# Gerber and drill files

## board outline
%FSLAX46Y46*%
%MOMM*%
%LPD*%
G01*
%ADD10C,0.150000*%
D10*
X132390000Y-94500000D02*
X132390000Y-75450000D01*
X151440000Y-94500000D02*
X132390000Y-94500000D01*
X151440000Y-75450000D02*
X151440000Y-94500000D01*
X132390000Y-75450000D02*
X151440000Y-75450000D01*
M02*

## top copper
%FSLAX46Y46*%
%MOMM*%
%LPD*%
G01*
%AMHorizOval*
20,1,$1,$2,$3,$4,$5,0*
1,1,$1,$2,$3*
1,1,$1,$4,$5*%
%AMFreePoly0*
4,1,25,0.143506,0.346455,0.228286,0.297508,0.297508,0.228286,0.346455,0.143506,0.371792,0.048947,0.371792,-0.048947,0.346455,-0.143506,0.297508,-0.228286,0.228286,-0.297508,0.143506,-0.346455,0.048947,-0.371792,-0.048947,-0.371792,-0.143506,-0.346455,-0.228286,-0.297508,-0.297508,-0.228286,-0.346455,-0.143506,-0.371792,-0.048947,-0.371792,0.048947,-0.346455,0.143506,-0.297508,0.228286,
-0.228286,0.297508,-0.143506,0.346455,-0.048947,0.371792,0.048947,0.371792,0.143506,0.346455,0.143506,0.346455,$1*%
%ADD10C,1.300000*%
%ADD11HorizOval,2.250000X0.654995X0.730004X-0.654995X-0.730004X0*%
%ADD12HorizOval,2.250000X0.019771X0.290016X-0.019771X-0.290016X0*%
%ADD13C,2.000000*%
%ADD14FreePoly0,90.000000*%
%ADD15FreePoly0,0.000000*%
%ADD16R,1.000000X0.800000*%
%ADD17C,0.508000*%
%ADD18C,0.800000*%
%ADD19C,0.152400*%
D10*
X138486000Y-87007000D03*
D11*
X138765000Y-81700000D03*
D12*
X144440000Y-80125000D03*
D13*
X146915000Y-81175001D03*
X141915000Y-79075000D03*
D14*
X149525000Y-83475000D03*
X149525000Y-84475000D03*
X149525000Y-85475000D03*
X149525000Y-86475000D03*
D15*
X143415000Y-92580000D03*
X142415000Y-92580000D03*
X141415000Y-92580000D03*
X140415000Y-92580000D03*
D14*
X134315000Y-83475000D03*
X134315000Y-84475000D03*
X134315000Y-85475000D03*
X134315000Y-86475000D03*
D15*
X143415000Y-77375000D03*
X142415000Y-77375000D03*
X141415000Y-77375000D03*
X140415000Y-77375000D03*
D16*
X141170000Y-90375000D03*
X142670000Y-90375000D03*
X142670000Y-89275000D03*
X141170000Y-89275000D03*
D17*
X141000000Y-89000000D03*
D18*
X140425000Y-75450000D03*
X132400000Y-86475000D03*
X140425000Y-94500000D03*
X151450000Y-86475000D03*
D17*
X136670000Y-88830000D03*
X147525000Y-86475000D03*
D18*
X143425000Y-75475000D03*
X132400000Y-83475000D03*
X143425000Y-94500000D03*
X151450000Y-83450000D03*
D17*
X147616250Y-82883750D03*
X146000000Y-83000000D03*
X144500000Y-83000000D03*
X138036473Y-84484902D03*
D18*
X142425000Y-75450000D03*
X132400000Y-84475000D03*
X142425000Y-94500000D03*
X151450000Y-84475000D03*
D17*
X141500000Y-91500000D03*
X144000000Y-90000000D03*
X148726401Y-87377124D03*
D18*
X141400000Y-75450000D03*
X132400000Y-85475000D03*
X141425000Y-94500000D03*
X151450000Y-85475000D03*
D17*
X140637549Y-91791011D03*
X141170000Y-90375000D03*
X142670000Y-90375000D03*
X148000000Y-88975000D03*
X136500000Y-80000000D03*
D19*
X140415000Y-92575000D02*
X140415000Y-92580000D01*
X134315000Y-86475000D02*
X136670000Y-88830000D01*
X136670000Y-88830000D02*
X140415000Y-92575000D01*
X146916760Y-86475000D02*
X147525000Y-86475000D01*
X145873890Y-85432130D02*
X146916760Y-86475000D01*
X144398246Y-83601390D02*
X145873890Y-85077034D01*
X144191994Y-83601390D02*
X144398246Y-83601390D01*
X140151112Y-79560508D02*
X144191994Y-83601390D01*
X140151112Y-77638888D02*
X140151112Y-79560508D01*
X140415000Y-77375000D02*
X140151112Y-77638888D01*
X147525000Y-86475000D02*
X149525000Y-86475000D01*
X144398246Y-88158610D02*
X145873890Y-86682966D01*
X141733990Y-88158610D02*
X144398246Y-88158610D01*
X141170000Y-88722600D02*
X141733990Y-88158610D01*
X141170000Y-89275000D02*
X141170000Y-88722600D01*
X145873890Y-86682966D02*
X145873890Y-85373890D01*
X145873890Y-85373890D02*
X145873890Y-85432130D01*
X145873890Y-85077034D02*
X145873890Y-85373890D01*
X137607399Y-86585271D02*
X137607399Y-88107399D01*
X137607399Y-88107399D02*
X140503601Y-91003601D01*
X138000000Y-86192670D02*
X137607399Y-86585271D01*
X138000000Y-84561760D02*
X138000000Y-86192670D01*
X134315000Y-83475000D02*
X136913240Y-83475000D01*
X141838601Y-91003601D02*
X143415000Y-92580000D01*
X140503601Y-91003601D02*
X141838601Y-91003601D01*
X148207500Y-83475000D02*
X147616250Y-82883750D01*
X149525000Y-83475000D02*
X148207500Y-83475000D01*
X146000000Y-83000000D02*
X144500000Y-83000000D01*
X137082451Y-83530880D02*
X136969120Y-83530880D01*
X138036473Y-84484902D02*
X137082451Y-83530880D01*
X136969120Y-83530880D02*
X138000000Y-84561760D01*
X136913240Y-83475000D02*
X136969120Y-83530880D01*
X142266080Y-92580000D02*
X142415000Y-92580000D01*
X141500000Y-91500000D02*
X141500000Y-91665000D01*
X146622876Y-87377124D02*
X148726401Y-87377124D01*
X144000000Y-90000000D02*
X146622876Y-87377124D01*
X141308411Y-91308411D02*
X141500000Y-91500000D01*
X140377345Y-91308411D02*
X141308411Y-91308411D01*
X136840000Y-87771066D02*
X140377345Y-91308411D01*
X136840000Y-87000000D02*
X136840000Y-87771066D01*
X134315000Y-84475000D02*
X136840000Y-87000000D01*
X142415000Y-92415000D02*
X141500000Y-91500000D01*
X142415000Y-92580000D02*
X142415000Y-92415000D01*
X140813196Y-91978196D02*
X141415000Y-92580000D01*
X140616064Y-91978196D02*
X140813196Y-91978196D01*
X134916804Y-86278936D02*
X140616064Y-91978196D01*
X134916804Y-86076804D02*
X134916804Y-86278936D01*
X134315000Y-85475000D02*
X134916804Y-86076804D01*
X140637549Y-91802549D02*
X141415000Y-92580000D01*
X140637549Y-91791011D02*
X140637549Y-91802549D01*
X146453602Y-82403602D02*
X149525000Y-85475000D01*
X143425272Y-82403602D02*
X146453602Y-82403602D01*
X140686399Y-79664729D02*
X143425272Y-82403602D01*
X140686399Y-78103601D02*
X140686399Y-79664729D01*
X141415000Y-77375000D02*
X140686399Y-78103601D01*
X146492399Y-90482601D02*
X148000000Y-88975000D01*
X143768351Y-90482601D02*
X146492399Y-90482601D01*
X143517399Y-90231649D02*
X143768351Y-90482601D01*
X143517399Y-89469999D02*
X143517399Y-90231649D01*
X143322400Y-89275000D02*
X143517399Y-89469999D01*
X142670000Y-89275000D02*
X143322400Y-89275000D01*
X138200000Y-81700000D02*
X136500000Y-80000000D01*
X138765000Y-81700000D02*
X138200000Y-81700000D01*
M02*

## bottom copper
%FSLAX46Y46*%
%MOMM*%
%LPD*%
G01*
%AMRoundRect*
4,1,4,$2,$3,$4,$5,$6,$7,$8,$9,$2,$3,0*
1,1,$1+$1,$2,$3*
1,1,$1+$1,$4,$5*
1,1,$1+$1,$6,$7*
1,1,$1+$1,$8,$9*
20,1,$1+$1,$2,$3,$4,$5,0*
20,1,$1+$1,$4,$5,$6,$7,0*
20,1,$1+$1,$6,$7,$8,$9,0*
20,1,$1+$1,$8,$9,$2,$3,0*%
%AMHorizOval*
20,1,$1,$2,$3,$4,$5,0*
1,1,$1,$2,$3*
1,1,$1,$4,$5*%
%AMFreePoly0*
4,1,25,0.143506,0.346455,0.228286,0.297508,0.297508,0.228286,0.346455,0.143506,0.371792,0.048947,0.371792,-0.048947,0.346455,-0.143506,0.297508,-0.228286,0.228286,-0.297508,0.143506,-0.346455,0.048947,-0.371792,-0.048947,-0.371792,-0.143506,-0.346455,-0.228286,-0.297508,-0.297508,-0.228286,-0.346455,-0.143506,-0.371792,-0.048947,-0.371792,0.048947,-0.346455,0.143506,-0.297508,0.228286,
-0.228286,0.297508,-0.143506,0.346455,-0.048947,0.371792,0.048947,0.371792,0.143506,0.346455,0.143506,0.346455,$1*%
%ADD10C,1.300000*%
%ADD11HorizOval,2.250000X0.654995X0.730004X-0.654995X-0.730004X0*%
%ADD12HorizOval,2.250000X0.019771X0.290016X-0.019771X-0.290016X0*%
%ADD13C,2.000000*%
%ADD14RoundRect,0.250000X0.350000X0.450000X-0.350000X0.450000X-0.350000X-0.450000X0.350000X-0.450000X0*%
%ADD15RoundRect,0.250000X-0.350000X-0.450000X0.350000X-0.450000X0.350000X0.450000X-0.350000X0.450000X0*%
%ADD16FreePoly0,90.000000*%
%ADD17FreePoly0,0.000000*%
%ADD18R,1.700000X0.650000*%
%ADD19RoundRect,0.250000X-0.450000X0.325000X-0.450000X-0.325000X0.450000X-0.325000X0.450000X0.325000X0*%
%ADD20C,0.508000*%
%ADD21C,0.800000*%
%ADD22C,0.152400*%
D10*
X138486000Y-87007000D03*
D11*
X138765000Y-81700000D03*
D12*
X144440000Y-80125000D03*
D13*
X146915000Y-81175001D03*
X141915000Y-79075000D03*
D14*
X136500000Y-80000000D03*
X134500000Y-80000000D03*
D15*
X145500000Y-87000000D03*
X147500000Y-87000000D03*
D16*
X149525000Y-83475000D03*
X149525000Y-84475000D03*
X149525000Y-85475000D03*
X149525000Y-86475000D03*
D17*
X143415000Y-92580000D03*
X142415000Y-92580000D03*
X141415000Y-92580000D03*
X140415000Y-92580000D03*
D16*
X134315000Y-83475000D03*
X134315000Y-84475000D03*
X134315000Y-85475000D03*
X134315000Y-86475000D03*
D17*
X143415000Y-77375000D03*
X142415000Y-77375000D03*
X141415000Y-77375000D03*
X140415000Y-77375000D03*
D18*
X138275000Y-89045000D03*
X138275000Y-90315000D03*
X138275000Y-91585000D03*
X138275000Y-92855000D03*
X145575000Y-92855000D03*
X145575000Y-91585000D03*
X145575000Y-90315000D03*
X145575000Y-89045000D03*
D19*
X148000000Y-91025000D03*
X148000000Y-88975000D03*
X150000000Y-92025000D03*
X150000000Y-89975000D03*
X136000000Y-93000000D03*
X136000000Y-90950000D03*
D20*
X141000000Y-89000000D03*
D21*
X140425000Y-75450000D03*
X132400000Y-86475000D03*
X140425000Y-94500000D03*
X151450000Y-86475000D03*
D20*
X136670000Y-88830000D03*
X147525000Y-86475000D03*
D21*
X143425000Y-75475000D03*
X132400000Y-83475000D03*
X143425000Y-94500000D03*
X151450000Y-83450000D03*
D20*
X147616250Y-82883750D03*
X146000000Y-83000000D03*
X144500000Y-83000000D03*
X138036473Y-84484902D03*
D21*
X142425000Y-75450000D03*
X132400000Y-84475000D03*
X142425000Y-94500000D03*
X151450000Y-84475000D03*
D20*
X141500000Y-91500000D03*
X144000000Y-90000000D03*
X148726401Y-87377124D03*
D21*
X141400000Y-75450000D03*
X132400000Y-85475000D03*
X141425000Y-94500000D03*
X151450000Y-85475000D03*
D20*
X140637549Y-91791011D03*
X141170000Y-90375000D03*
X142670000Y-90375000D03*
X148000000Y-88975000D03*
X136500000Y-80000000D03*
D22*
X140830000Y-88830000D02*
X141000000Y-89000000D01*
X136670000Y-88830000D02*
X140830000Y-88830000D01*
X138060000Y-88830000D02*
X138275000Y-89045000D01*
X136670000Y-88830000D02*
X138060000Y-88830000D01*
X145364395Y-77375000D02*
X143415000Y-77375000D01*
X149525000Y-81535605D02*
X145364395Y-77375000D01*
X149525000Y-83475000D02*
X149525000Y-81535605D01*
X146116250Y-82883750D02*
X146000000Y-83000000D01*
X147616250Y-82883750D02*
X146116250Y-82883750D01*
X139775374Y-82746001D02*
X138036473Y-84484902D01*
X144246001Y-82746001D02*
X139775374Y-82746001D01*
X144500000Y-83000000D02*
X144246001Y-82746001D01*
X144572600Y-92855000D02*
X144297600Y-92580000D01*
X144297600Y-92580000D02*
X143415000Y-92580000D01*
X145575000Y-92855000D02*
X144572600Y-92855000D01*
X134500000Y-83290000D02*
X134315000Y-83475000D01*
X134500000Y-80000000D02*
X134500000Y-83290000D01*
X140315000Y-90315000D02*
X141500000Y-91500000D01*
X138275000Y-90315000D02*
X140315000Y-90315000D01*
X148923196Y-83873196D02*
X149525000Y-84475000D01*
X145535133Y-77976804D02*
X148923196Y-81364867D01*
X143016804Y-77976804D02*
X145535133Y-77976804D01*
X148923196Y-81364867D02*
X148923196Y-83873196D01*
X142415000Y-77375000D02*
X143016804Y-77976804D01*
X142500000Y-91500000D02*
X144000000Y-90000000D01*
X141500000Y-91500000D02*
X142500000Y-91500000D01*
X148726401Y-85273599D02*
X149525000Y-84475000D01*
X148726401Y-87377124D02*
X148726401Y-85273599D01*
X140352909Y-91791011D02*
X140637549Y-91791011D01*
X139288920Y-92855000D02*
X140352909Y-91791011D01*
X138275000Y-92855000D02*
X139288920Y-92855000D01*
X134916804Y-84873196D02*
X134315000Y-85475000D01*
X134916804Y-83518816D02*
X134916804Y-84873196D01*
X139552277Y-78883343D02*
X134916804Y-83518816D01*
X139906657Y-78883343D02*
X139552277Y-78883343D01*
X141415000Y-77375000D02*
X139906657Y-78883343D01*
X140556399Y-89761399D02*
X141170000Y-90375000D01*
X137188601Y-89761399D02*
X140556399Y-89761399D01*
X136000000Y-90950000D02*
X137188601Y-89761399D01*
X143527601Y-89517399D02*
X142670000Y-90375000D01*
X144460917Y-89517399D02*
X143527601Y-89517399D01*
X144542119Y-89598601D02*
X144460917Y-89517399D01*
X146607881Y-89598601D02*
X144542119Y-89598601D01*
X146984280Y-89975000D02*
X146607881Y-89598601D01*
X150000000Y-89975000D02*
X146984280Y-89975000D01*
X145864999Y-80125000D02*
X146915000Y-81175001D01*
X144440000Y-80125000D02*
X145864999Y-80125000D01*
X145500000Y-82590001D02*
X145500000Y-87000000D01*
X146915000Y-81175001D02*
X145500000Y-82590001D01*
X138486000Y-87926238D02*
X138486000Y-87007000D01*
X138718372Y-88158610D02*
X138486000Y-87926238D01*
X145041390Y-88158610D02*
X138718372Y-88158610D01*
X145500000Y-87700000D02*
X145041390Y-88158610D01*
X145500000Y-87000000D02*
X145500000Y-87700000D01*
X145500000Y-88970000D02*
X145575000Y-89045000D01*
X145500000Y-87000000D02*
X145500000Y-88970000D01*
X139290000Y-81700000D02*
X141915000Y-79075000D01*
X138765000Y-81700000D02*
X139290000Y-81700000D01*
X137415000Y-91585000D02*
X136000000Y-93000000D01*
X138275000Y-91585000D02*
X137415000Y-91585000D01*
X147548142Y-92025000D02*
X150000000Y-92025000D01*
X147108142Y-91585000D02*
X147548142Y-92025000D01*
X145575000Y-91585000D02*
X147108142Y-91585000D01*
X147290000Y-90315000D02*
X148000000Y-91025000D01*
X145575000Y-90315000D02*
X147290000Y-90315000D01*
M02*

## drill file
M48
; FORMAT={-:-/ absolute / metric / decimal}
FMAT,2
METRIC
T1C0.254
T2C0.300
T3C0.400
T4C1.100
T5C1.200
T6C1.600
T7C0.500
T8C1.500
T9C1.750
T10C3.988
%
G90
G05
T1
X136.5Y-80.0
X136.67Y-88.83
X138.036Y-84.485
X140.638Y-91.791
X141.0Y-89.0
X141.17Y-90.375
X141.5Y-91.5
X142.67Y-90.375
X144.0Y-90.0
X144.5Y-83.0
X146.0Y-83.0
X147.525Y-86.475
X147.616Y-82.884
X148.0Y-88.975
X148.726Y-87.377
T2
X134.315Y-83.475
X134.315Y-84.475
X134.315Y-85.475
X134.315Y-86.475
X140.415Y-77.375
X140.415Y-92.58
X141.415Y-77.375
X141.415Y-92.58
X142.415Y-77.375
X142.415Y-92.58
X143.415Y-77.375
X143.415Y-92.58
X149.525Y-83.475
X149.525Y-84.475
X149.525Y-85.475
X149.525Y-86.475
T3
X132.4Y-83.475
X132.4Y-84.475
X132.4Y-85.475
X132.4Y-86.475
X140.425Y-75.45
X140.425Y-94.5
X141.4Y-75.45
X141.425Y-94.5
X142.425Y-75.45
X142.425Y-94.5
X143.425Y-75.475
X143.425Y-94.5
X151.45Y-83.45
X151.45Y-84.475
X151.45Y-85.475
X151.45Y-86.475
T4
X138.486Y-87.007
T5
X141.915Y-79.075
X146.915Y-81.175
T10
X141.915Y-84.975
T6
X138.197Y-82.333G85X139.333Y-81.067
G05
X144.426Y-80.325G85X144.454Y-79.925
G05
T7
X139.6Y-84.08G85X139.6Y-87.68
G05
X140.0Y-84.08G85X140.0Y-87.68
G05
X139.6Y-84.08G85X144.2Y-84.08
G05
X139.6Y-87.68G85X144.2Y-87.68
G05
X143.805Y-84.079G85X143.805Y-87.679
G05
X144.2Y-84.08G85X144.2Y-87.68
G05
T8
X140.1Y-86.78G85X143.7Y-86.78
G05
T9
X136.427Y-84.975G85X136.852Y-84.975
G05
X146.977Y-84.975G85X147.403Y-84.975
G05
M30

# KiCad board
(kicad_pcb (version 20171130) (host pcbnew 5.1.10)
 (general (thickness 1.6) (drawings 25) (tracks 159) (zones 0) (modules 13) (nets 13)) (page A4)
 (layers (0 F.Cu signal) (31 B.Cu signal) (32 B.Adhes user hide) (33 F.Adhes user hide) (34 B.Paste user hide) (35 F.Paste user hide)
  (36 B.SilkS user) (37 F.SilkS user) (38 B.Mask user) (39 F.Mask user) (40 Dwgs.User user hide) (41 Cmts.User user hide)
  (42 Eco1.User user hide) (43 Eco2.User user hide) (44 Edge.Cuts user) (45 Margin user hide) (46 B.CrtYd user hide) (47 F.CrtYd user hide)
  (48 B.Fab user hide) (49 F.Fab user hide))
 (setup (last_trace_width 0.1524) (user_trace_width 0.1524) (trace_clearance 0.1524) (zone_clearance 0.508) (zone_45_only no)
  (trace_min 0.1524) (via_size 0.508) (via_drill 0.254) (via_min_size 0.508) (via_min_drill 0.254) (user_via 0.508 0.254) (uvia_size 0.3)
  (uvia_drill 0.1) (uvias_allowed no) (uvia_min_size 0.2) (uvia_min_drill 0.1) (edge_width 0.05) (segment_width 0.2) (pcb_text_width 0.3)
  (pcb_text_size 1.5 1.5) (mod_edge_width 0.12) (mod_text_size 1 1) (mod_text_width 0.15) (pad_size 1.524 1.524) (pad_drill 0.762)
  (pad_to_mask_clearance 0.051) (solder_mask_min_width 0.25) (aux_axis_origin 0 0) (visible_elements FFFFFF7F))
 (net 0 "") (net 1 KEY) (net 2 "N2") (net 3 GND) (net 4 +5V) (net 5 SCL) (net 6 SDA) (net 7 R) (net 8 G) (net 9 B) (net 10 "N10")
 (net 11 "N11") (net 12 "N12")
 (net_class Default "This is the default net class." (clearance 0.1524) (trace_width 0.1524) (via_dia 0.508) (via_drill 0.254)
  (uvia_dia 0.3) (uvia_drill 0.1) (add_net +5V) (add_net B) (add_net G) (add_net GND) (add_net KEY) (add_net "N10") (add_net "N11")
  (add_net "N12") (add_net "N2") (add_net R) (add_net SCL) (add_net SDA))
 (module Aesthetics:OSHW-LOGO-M (layer F.Cu) (at 147.5 91)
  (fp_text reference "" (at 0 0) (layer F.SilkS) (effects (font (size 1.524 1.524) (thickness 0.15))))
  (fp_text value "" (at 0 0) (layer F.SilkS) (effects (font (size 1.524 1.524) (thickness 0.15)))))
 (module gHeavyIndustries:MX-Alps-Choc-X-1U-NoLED (layer F.Cu) (at 141.915 84.975)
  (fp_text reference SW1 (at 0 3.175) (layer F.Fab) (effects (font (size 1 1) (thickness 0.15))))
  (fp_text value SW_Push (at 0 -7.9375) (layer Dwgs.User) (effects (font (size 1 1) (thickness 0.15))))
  (pad 1 thru_hole circle (at -3.429 2.032) (size 1.3 1.3) (drill 1.1) (layers *.Cu *.Mask) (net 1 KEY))
  (pad "" np_thru_hole oval (at -2.315 0.905) (size 0.5 4.1) (drill oval 0.5 4.1) (layers *.Cu *.Mask))
  (pad "" np_thru_hole oval (at 1.89 0.90416) (size 0.5 4.1) (drill oval 0.5 4.1) (layers *.Cu *.Mask))
  (pad "" np_thru_hole oval (at 2.285 0.905) (size 0.5 4.1) (drill oval 0.5 4.1) (layers *.Cu *.Mask))
  (pad "" np_thru_hole oval (at -0.015 2.705) (size 5.1 0.5) (drill oval 5.1 0.5) (layers *.Cu *.Mask))
  (pad "" np_thru_hole oval (at -0.015 -0.895) (size 5.1 0.5) (drill oval 5.1 0.5) (layers *.Cu *.Mask))
  (pad "" np_thru_hole oval (at -1.915 0.905) (size 0.5 4.1) (drill oval 0.5 4.1) (layers *.Cu *.Mask))
  (pad "" np_thru_hole oval (at -0.015 1.805) (size 5.1 1.5) (drill oval 5.1 1.5) (layers *.Cu *.Mask))
  (pad 2 thru_hole oval (at -3.15 -3.275 48.1) (size 4.211556 2.25) (drill oval 3.3 1.6) (layers *.Cu *.Mask) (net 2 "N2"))
  (pad 1 thru_hole oval (at 2.525 -4.85 86.1) (size 2.831378 2.25) (drill oval 2 1.6) (layers *.Cu *.Mask) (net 1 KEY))
  (pad "" np_thru_hole oval (at 5.275 0 90) (size 1.75 2.175) (drill oval 1.75 2.175) (layers *.Cu *.Mask))
  (pad "" np_thru_hole oval (at -5.275 0 90) (size 1.75 2.175) (drill oval 1.75 2.175) (layers *.Cu *.Mask))
  (pad "" np_thru_hole circle (at 0 0) (size 3.9878 3.9878) (drill 3.9878) (layers *.Cu *.Mask))
  (pad 1 thru_hole circle (at 5 -3.799999) (size 2 2) (drill 1.2) (layers *.Cu *.Mask) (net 1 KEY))
  (pad 2 thru_hole circle (at 0 -5.9) (size 2 2) (drill 1.2) (layers *.Cu *.Mask) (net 2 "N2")))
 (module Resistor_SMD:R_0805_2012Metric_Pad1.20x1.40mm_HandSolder (layer B.Cu) (at 135.5 80 180)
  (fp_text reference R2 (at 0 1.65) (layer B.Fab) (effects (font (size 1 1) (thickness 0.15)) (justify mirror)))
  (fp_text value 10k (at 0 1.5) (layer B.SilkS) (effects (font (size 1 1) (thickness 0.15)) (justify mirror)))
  (pad 1 smd roundrect (at -1 0 180) (size 1.2 1.4) (layers B.Cu B.Paste B.Mask) (roundrect_rratio 0.208333) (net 2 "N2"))
  (pad 2 smd roundrect (at 1 0 180) (size 1.2 1.4) (layers B.Cu B.Paste B.Mask) (roundrect_rratio 0.208333) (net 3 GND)))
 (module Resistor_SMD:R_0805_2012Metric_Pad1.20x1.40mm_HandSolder (layer B.Cu) (at 146.5 87)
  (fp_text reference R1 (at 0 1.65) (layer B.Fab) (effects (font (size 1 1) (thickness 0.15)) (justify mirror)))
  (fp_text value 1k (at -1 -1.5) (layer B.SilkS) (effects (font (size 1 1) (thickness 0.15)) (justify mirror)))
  (pad 1 smd roundrect (at -1 0) (size 1.2 1.4) (layers B.Cu B.Paste B.Mask) (roundrect_rratio 0.208333) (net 1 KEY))
  (pad 2 smd roundrect (at 1 0) (size 1.2 1.4) (layers B.Cu B.Paste B.Mask) (roundrect_rratio 0.208333) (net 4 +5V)))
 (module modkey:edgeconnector (layer F.Cu) (at 151.525 84.975 90)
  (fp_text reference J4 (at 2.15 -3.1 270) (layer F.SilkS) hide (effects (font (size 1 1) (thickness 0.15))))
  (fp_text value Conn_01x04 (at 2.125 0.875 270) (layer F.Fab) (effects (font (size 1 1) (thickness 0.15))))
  (pad 4 thru_hole custom (at 1.5 -2 90) (size 0.75 0.75) (drill 0.3) (layers *.Cu *.Mask) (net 3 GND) (zone_connect 0)
   (options (clearance outline) (anchor circle)) (primitives))
  (pad 3 thru_hole custom (at 0.5 -2 90) (size 0.75 0.75) (drill 0.3) (layers *.Cu *.Mask) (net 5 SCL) (zone_connect 0)
   (options (clearance outline) (anchor circle)) (primitives))
  (pad 2 thru_hole custom (at -0.5 -2 90) (size 0.75 0.75) (drill 0.3) (layers *.Cu *.Mask) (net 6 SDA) (zone_connect 0)
   (options (clearance outline) (anchor circle)) (primitives))
  (pad 1 thru_hole custom (at -1.5 -2 90) (size 0.75 0.75) (drill 0.3) (layers *.Cu *.Mask) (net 4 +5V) (zone_connect 0)
   (options (clearance outline) (anchor circle)) (primitives)))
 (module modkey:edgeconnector (layer F.Cu) (at 141.915 94.58)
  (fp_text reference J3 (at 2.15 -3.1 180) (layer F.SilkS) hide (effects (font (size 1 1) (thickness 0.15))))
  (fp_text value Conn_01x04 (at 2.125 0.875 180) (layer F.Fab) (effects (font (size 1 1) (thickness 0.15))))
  (pad 4 thru_hole custom (at 1.5 -2) (size 0.75 0.75) (drill 0.3) (layers *.Cu *.Mask) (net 3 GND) (zone_connect 0)
   (options (clearance outline) (anchor circle)) (primitives))
  (pad 3 thru_hole custom (at 0.5 -2) (size 0.75 0.75) (drill 0.3) (layers *.Cu *.Mask) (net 5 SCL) (zone_connect 0)
   (options (clearance outline) (anchor circle)) (primitives))
  (pad 2 thru_hole custom (at -0.5 -2) (size 0.75 0.75) (drill 0.3) (layers *.Cu *.Mask) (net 6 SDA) (zone_connect 0)
   (options (clearance outline) (anchor circle)) (primitives))
  (pad 1 thru_hole custom (at -1.5 -2) (size 0.75 0.75) (drill 0.3) (layers *.Cu *.Mask) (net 4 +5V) (zone_connect 0)
   (options (clearance outline) (anchor circle)) (primitives)))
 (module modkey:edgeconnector (layer B.Cu) (at 132.315 84.975 90)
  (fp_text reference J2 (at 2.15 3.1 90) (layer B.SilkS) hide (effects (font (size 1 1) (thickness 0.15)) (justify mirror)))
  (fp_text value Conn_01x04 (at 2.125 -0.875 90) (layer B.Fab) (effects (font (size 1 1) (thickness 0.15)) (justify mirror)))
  (pad 4 thru_hole custom (at 1.5 2 90) (size 0.75 0.75) (drill 0.3) (layers *.Cu *.Mask) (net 3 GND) (zone_connect 0)
   (options (clearance outline) (anchor circle)) (primitives))
  (pad 3 thru_hole custom (at 0.5 2 90) (size 0.75 0.75) (drill 0.3) (layers *.Cu *.Mask) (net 5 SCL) (zone_connect 0)
   (options (clearance outline) (anchor circle)) (primitives))
  (pad 2 thru_hole custom (at -0.5 2 90) (size 0.75 0.75) (drill 0.3) (layers *.Cu *.Mask) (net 6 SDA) (zone_connect 0)
   (options (clearance outline) (anchor circle)) (primitives))
  (pad 1 thru_hole custom (at -1.5 2 90) (size 0.75 0.75) (drill 0.3) (layers *.Cu *.Mask) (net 4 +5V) (zone_connect 0)
   (options (clearance outline) (anchor circle)) (primitives)))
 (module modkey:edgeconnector (layer B.Cu) (at 141.915 75.375)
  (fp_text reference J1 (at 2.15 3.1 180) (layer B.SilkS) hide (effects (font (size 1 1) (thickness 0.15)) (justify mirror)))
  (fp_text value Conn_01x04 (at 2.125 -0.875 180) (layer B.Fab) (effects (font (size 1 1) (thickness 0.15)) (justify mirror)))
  (pad 4 thru_hole custom (at 1.5 2) (size 0.75 0.75) (drill 0.3) (layers *.Cu *.Mask) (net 3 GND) (zone_connect 0)
   (options (clearance outline) (anchor circle)) (primitives))
  (pad 3 thru_hole custom (at 0.5 2) (size 0.75 0.75) (drill 0.3) (layers *.Cu *.Mask) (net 5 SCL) (zone_connect 0)
   (options (clearance outline) (anchor circle)) (primitives))
  (pad 2 thru_hole custom (at -0.5 2) (size 0.75 0.75) (drill 0.3) (layers *.Cu *.Mask) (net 6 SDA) (zone_connect 0)
   (options (clearance outline) (anchor circle)) (primitives))
  (pad 1 thru_hole custom (at -1.5 2) (size 0.75 0.75) (drill 0.3) (layers *.Cu *.Mask) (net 4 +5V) (zone_connect 0)
   (options (clearance outline) (anchor circle)) (primitives)))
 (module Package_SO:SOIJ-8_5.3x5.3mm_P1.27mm (layer B.Cu) (at 141.925 90.95 180)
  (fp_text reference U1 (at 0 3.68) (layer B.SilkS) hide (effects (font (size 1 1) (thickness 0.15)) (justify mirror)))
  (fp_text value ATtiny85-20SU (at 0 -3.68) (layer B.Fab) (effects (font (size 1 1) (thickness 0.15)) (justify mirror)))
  (pad 8 smd rect (at 3.65 1.905 180) (size 1.7 0.65) (layers B.Cu B.Paste B.Mask) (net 4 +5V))
  (pad 7 smd rect (at 3.65 0.635 180) (size 1.7 0.65) (layers B.Cu B.Paste B.Mask) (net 5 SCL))
  (pad 6 smd rect (at 3.65 -0.635 180) (size 1.7 0.65) (layers B.Cu B.Paste B.Mask) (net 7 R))
  (pad 5 smd rect (at 3.65 -1.905 180) (size 1.7 0.65) (layers B.Cu B.Paste B.Mask) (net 6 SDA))
  (pad 4 smd rect (at -3.65 -1.905 180) (size 1.7 0.65) (layers B.Cu B.Paste B.Mask) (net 3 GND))
  (pad 3 smd rect (at -3.65 -0.635 180) (size 1.7 0.65) (layers B.Cu B.Paste B.Mask) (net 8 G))
  (pad 2 smd rect (at -3.65 0.635 180) (size 1.7 0.65) (layers B.Cu B.Paste B.Mask) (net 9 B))
  (pad 1 smd rect (at -3.65 1.905 180) (size 1.7 0.65) (layers B.Cu B.Paste B.Mask) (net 1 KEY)))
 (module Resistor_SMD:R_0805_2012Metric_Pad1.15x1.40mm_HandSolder (layer B.Cu) (at 148 90 270)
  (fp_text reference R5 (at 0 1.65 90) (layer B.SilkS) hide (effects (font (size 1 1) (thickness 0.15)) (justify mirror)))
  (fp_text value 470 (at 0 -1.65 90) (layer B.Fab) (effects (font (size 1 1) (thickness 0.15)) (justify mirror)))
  (pad 2 smd roundrect (at 1.025 0 270) (size 1.15 1.4) (layers B.Cu B.Paste B.Mask) (roundrect_rratio 0.217391) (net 9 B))
  (pad 1 smd roundrect (at -1.025 0 270) (size 1.15 1.4) (layers B.Cu B.Paste B.Mask) (roundrect_rratio 0.217391) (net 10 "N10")))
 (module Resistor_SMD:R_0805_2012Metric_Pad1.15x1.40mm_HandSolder (layer B.Cu) (at 150 91 270)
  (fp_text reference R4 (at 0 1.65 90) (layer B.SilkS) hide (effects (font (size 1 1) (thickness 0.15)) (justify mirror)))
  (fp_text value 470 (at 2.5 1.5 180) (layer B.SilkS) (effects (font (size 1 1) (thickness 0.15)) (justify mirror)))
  (pad 2 smd roundrect (at 1.025 0 270) (size 1.15 1.4) (layers B.Cu B.Paste B.Mask) (roundrect_rratio 0.217391) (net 8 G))
  (pad 1 smd roundrect (at -1.025 0 270) (size 1.15 1.4) (layers B.Cu B.Paste B.Mask) (roundrect_rratio 0.217391) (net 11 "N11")))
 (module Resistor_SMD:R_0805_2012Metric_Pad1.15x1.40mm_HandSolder (layer B.Cu) (at 136 91.975 270)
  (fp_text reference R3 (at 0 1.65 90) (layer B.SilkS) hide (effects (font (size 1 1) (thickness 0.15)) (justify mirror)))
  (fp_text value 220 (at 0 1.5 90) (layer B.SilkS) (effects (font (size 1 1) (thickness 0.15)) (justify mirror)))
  (pad 2 smd roundrect (at 1.025 0 270) (size 1.15 1.4) (layers B.Cu B.Paste B.Mask) (roundrect_rratio 0.217391) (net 7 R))
  (pad 1 smd roundrect (at -1.025 0 270) (size 1.15 1.4) (layers B.Cu B.Paste B.Mask) (roundrect_rratio 0.217391) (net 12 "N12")))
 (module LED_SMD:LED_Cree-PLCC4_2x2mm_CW (layer F.Cu) (at 141.92 89.825)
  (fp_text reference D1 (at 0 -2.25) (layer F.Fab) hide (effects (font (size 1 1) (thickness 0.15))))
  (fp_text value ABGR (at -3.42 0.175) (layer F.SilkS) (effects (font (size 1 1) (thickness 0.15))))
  (pad 4 smd rect (at -0.75 0.55) (size 1 0.8) (layers F.Cu F.Paste F.Mask) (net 12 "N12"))
  (pad 3 smd rect (at 0.75 0.55) (size 1 0.8) (layers F.Cu F.Paste F.Mask) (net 11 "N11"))
  (pad 2 smd rect (at 0.75 -0.55) (size 1 0.8) (layers F.Cu F.Paste F.Mask) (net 10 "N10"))
  (pad 1 smd rect (at -0.75 -0.55) (size 1 0.8) (layers F.Cu F.Paste F.Mask) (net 4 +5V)))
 (gr_line (start 132.39 94.5) (end 132.39 75.45) (layer Edge.Cuts) (width 0.15))
 (gr_line (start 151.44 94.5) (end 132.39 94.5) (layer Edge.Cuts) (width 0.15))
 (gr_line (start 151.44 75.45) (end 151.44 94.5) (layer Edge.Cuts) (width 0.15))
 (gr_line (start 132.39 75.45) (end 151.44 75.45) (layer Edge.Cuts) (width 0.15))
 (via (at 141 89) (size 0.508) (drill 0.254) (layers F.Cu B.Cu) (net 4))
 (via (at 140.425 75.45) (size 0.8) (drill 0.4) (layers F.Cu B.Cu) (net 4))
 (via (at 132.4 86.475) (size 0.8) (drill 0.4) (layers F.Cu B.Cu) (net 4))
 (via (at 140.425 94.5) (size 0.8) (drill 0.4) (layers F.Cu B.Cu) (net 4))
 (via (at 151.45 86.475) (size 0.8) (drill 0.4) (layers F.Cu B.Cu) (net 4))
 (segment (start 140.415 92.575) (end 140.415 92.58) (width 0.1524) (layer F.Cu) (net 4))
 (segment (start 134.315 86.475) (end 136.67 88.83) (width 0.1524) (layer F.Cu) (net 4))
 (segment (start 136.67 88.83) (end 140.415 92.575) (width 0.1524) (layer F.Cu) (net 4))
 (via (at 136.67 88.83) (size 0.508) (drill 0.254) (layers F.Cu B.Cu) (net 4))
 (segment (start 140.83 88.83) (end 141 89) (width 0.1524) (layer B.Cu) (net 4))
 (segment (start 136.67 88.83) (end 140.83 88.83) (width 0.1524) (layer B.Cu) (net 4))
 (segment (start 138.06 88.83) (end 138.275 89.045) (width 0.1524) (layer B.Cu) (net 4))
 (segment (start 136.67 88.83) (end 138.06 88.83) (width 0.1524) (layer B.Cu) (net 4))
 (segment (start 146.91676 86.475) (end 147.525 86.475) (width 0.1524) (layer F.Cu) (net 4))
 (segment (start 145.87389 85.43213) (end 146.91676 86.475) (width 0.1524) (layer F.Cu) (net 4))
 (segment (start 144.398246 83.60139) (end 145.87389 85.077034) (width 0.1524) (layer F.Cu) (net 4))
 (segment (start 144.191994 83.60139) (end 144.398246 83.60139) (width 0.1524) (layer F.Cu) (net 4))
 (segment (start 140.151112 79.560508) (end 144.191994 83.60139) (width 0.1524) (layer F.Cu) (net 4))
 (segment (start 140.151112 77.638888) (end 140.151112 79.560508) (width 0.1524) (layer F.Cu) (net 4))
 (segment (start 140.415 77.375) (end 140.151112 77.638888) (width 0.1524) (layer F.Cu) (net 4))
 (segment (start 147.525 86.475) (end 149.525 86.475) (width 0.1524) (layer F.Cu) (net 4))
 (via (at 147.525 86.475) (size 0.508) (drill 0.254) (layers F.Cu B.Cu) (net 4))
 (segment (start 144.398246 88.15861) (end 145.87389 86.682966) (width 0.1524) (layer F.Cu) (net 4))
 (segment (start 141.73399 88.15861) (end 144.398246 88.15861) (width 0.1524) (layer F.Cu) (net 4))
 (segment (start 141.17 88.7226) (end 141.73399 88.15861) (width 0.1524) (layer F.Cu) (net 4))
 (segment (start 141.17 89.275) (end 141.17 88.7226) (width 0.1524) (layer F.Cu) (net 4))
 (segment (start 145.87389 86.682966) (end 145.87389 85.37389) (width 0.1524) (layer F.Cu) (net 4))
 (segment (start 145.87389 85.37389) (end 145.87389 85.43213) (width 0.1524) (layer F.Cu) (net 4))
 (segment (start 145.87389 85.077034) (end 145.87389 85.37389) (width 0.1524) (layer F.Cu) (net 4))
 (via (at 143.425 75.475) (size 0.8) (drill 0.4) (layers F.Cu B.Cu) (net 3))
 (via (at 132.4 83.475) (size 0.8) (drill 0.4) (layers F.Cu B.Cu) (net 3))
 (via (at 143.425 94.5) (size 0.8) (drill 0.4) (layers F.Cu B.Cu) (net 3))
 (via (at 151.45 83.45) (size 0.8) (drill 0.4) (layers F.Cu B.Cu) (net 3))
 (segment (start 137.607399 86.585271) (end 137.607399 88.107399) (width 0.1524) (layer F.Cu) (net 3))
 (segment (start 137.607399 88.107399) (end 140.503601 91.003601) (width 0.1524) (layer F.Cu) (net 3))
 (segment (start 138 86.19267) (end 137.607399 86.585271) (width 0.1524) (layer F.Cu) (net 3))
 (segment (start 138 84.56176) (end 138 86.19267) (width 0.1524) (layer F.Cu) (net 3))
 (segment (start 134.315 83.475) (end 136.91324 83.475) (width 0.1524) (layer F.Cu) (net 3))
 (segment (start 141.838601 91.003601) (end 143.415 92.58) (width 0.1524) (layer F.Cu) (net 3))
 (segment (start 140.503601 91.003601) (end 141.838601 91.003601) (width 0.1524) (layer F.Cu) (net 3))
 (segment (start 145.364395 77.375) (end 143.415 77.375) (width 0.1524) (layer B.Cu) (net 3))
 (segment (start 149.525 81.535605) (end 145.364395 77.375) (width 0.1524) (layer B.Cu) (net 3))
 (segment (start 149.525 83.475) (end 149.525 81.535605) (width 0.1524) (layer B.Cu) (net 3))
 (via (at 147.61625 82.88375) (size 0.508) (drill 0.254) (layers F.Cu B.Cu) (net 3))
 (segment (start 148.2075 83.475) (end 147.61625 82.88375) (width 0.1524) (layer F.Cu) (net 3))
 (segment (start 149.525 83.475) (end 148.2075 83.475) (width 0.1524) (layer F.Cu) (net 3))
 (via (at 146 83) (size 0.508) (drill 0.254) (layers F.Cu B.Cu) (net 3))
 (segment (start 146.11625 82.88375) (end 146 83) (width 0.1524) (layer B.Cu) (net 3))
 (segment (start 147.61625 82.88375) (end 146.11625 82.88375) (width 0.1524) (layer B.Cu) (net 3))
 (via (at 144.5 83) (size 0.508) (drill 0.254) (layers F.Cu B.Cu) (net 3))
 (segment (start 146 83) (end 144.5 83) (width 0.1524) (layer F.Cu) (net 3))
 (via (at 138.036473 84.484902) (size 0.508) (drill 0.254) (layers F.Cu B.Cu) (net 3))
 (segment (start 139.775374 82.746001) (end 138.036473 84.484902) (width 0.1524) (layer B.Cu) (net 3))
 (segment (start 144.246001 82.746001) (end 139.775374 82.746001) (width 0.1524) (layer B.Cu) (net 3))
 (segment (start 144.5 83) (end 144.246001 82.746001) (width 0.1524) (layer B.Cu) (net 3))
 (segment (start 137.082451 83.53088) (end 136.96912 83.53088) (width 0.1524) (layer F.Cu) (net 3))
 (segment (start 138.036473 84.484902) (end 137.082451 83.53088) (width 0.1524) (layer F.Cu) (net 3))
 (segment (start 136.96912 83.53088) (end 138 84.56176) (width 0.1524) (layer F.Cu) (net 3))
 (segment (start 136.91324 83.475) (end 136.96912 83.53088) (width 0.1524) (layer F.Cu) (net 3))
 (segment (start 144.5726 92.855) (end 144.2976 92.58) (width 0.1524) (layer B.Cu) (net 3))
 (segment (start 144.2976 92.58) (end 143.415 92.58) (width 0.1524) (layer B.Cu) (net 3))
 (segment (start 145.575 92.855) (end 144.5726 92.855) (width 0.1524) (layer B.Cu) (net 3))
 (segment (start 134.5 83.29) (end 134.315 83.475) (width 0.1524) (layer B.Cu) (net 3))
 (segment (start 134.5 80) (end 134.5 83.29) (width 0.1524) (layer B.Cu) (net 3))
 (via (at 142.425 75.45) (size 0.8) (drill 0.4) (layers F.Cu B.Cu) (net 5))
 (via (at 132.4 84.475) (size 0.8) (drill 0.4) (layers F.Cu B.Cu) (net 5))
 (via (at 142.425 94.5) (size 0.8) (drill 0.4) (layers F.Cu B.Cu) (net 5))
 (via (at 151.45 84.475) (size 0.8) (drill 0.4) (layers F.Cu B.Cu) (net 5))
 (segment (start 142.26608 92.58) (end 142.415 92.58) (width 0.1524) (layer F.Cu) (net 5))
 (via (at 141.5 91.5) (size 0.508) (drill 0.254) (layers F.Cu B.Cu) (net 5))
 (segment (start 140.315 90.315) (end 141.5 91.5) (width 0.1524) (layer B.Cu) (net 5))
 (segment (start 138.275 90.315) (end 140.315 90.315) (width 0.1524) (layer B.Cu) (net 5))
 (segment (start 141.5 91.5) (end 141.5 91.665) (width 0.1524) (layer F.Cu) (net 5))
 (segment (start 148.923196 83.873196) (end 149.525 84.475) (width 0.1524) (layer B.Cu) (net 5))
 (segment (start 145.535133 77.976804) (end 148.923196 81.364867) (width 0.1524) (layer B.Cu) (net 5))
 (segment (start 143.016804 77.976804) (end 145.535133 77.976804) (width 0.1524) (layer B.Cu) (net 5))
 (segment (start 148.923196 81.364867) (end 148.923196 83.873196) (width 0.1524) (layer B.Cu) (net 5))
 (segment (start 142.415 77.375) (end 143.016804 77.976804) (width 0.1524) (layer B.Cu) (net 5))
 (via (at 144 90) (size 0.508) (drill 0.254) (layers F.Cu B.Cu) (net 5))
 (segment (start 142.5 91.5) (end 144 90) (width 0.1524) (layer B.Cu) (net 5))
 (segment (start 141.5 91.5) (end 142.5 91.5) (width 0.1524) (layer B.Cu) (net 5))
 (via (at 148.726401 87.377124) (size 0.508) (drill 0.254) (layers F.Cu B.Cu) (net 5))
 (segment (start 146.622876 87.377124) (end 148.726401 87.377124) (width 0.1524) (layer F.Cu) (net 5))
 (segment (start 144 90) (end 146.622876 87.377124) (width 0.1524) (layer F.Cu) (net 5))
 (segment (start 148.726401 85.273599) (end 149.525 84.475) (width 0.1524) (layer B.Cu) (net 5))
 (segment (start 148.726401 87.377124) (end 148.726401 85.273599) (width 0.1524) (layer B.Cu) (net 5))
 (segment (start 141.308411 91.308411) (end 141.5 91.5) (width 0.1524) (layer F.Cu) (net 5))
 (segment (start 140.377345 91.308411) (end 141.308411 91.308411) (width 0.1524) (layer F.Cu) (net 5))
 (segment (start 136.84 87.771066) (end 140.377345 91.308411) (width 0.1524) (layer F.Cu) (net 5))
 (segment (start 136.84 87) (end 136.84 87.771066) (width 0.1524) (layer F.Cu) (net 5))
 (segment (start 134.315 84.475) (end 136.84 87) (width 0.1524) (layer F.Cu) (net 5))
 (segment (start 142.415 92.415) (end 141.5 91.5) (width 0.1524) (layer F.Cu) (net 5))
 (segment (start 142.415 92.58) (end 142.415 92.415) (width 0.1524) (layer F.Cu) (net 5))
 (via (at 141.4 75.45) (size 0.8) (drill 0.4) (layers F.Cu B.Cu) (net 6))
 (via (at 132.4 85.475) (size 0.8) (drill 0.4) (layers F.Cu B.Cu) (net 6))
 (via (at 141.425 94.5) (size 0.8) (drill 0.4) (layers F.Cu B.Cu) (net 6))
 (via (at 151.45 85.475) (size 0.8) (drill 0.4) (layers F.Cu B.Cu) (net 6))
 (segment (start 140.813196 91.978196) (end 141.415 92.58) (width 0.1524) (layer F.Cu) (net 6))
 (segment (start 140.616064 91.978196) (end 140.813196 91.978196) (width 0.1524) (layer F.Cu) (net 6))
 (segment (start 134.916804 86.278936) (end 140.616064 91.978196) (width 0.1524) (layer F.Cu) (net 6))
 (segment (start 134.916804 86.076804) (end 134.916804 86.278936) (width 0.1524) (layer F.Cu) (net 6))
 (segment (start 134.315 85.475) (end 134.916804 86.076804) (width 0.1524) (layer F.Cu) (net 6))
 (via (at 140.637549 91.791011) (size 0.508) (drill 0.254) (layers F.Cu B.Cu) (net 6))
 (segment (start 140.352909 91.791011) (end 140.637549 91.791011) (width 0.1524) (layer B.Cu) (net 6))
 (segment (start 139.28892 92.855) (end 140.352909 91.791011) (width 0.1524) (layer B.Cu) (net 6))
 (segment (start 138.275 92.855) (end 139.28892 92.855) (width 0.1524) (layer B.Cu) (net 6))
 (segment (start 140.637549 91.802549) (end 141.415 92.58) (width 0.1524) (layer F.Cu) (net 6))
 (segment (start 140.637549 91.791011) (end 140.637549 91.802549) (width 0.1524) (layer F.Cu) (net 6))
 (segment (start 146.453602 82.403602) (end 149.525 85.475) (width 0.1524) (layer F.Cu) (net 6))
 (segment (start 143.425272 82.403602) (end 146.453602 82.403602) (width 0.1524) (layer F.Cu) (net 6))
 (segment (start 140.686399 79.664729) (end 143.425272 82.403602) (width 0.1524) (layer F.Cu) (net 6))
 (segment (start 140.686399 78.103601) (end 140.686399 79.664729) (width 0.1524) (layer F.Cu) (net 6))
 (segment (start 141.415 77.375) (end 140.686399 78.103601) (width 0.1524) (layer F.Cu) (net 6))
 (segment (start 134.916804 84.873196) (end 134.315 85.475) (width 0.1524) (layer B.Cu) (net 6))
 (segment (start 134.916804 83.518816) (end 134.916804 84.873196) (width 0.1524) (layer B.Cu) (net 6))
 (segment (start 139.552277 78.883343) (end 134.916804 83.518816) (width 0.1524) (layer B.Cu) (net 6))
 (segment (start 139.906657 78.883343) (end 139.552277 78.883343) (width 0.1524) (layer B.Cu) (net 6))
 (segment (start 141.415 77.375) (end 139.906657 78.883343) (width 0.1524) (layer B.Cu) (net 6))
 (via (at 141.17 90.375) (size 0.508) (drill 0.254) (layers F.Cu B.Cu) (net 12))
 (segment (start 140.556399 89.761399) (end 141.17 90.375) (width 0.1524) (layer B.Cu) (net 12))
 (segment (start 137.188601 89.761399) (end 140.556399 89.761399) (width 0.1524) (layer B.Cu) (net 12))
 (segment (start 136 90.95) (end 137.188601 89.761399) (width 0.1524) (layer B.Cu) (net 12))
 (via (at 142.67 90.375) (size 0.508) (drill 0.254) (layers F.Cu B.Cu) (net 11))
 (segment (start 143.527601 89.517399) (end 142.67 90.375) (width 0.1524) (layer B.Cu) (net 11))
 (segment (start 144.460917 89.517399) (end 143.527601 89.517399) (width 0.1524) (layer B.Cu) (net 11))
 (segment (start 144.542119 89.598601) (end 144.460917 89.517399) (width 0.1524) (layer B.Cu) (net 11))
 (segment (start 146.607881 89.598601) (end 144.542119 89.598601) (width 0.1524) (layer B.Cu) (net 11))
 (segment (start 146.98428 89.975) (end 146.607881 89.598601) (width 0.1524) (layer B.Cu) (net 11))
 (segment (start 150 89.975) (end 146.98428 89.975) (width 0.1524) (layer B.Cu) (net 11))
 (segment (start 146.492399 90.482601) (end 148 88.975) (width 0.1524) (layer F.Cu) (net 10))
 (segment (start 143.768351 90.482601) (end 146.492399 90.482601) (width 0.1524) (layer F.Cu) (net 10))
 (segment (start 143.517399 90.231649) (end 143.768351 90.482601) (width 0.1524) (layer F.Cu) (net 10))
 (segment (start 143.517399 89.469999) (end 143.517399 90.231649) (width 0.1524) (layer F.Cu) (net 10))
 (via (at 148 88.975) (size 0.508) (drill 0.254) (layers F.Cu B.Cu) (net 10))
 (segment (start 143.3224 89.275) (end 143.517399 89.469999) (width 0.1524) (layer F.Cu) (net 10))
 (segment (start 142.67 89.275) (end 143.3224 89.275) (width 0.1524) (layer F.Cu) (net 10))
 (segment (start 145.864999 80.125) (end 146.915 81.175001) (width 0.1524) (layer B.Cu) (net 1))
 (segment (start 144.44 80.125) (end 145.864999 80.125) (width 0.1524) (layer B.Cu) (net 1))
 (segment (start 145.5 82.590001) (end 145.5 87) (width 0.1524) (layer B.Cu) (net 1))
 (segment (start 146.915 81.175001) (end 145.5 82.590001) (width 0.1524) (layer B.Cu) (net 1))
 (segment (start 138.486 87.926238) (end 138.486 87.007) (width 0.1524) (layer B.Cu) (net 1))
 (segment (start 138.718372 88.15861) (end 138.486 87.926238) (width 0.1524) (layer B.Cu) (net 1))
 (segment (start 145.04139 88.15861) (end 138.718372 88.15861) (width 0.1524) (layer B.Cu) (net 1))
 (segment (start 145.5 87.7) (end 145.04139 88.15861) (width 0.1524) (layer B.Cu) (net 1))
 (segment (start 145.5 87) (end 145.5 87.7) (width 0.1524) (layer B.Cu) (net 1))
 (segment (start 145.5 88.97) (end 145.575 89.045) (width 0.1524) (layer B.Cu) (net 1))
 (segment (start 145.5 87) (end 145.5 88.97) (width 0.1524) (layer B.Cu) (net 1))
 (segment (start 139.29 81.7) (end 141.915 79.075) (width 0.1524) (layer B.Cu) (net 2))
 (segment (start 138.765 81.7) (end 139.29 81.7) (width 0.1524) (layer B.Cu) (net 2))
 (via (at 136.5 80) (size 0.508) (drill 0.254) (layers F.Cu B.Cu) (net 2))
 (segment (start 138.2 81.7) (end 136.5 80) (width 0.1524) (layer F.Cu) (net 2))
 (segment (start 138.765 81.7) (end 138.2 81.7) (width 0.1524) (layer F.Cu) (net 2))
 (segment (start 137.415 91.585) (end 136 93) (width 0.1524) (layer B.Cu) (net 7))
 (segment (start 138.275 91.585) (end 137.415 91.585) (width 0.1524) (layer B.Cu) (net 7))
 (segment (start 147.548142 92.025) (end 150 92.025) (width 0.1524) (layer B.Cu) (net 8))
 (segment (start 147.108142 91.585) (end 147.548142 92.025) (width 0.1524) (layer B.Cu) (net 8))
 (segment (start 145.575 91.585) (end 147.108142 91.585) (width 0.1524) (layer B.Cu) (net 8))
 (segment (start 147.29 90.315) (end 148 91.025) (width 0.1524) (layer B.Cu) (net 9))
 (segment (start 145.575 90.315) (end 147.29 90.315) (width 0.1524) (layer B.Cu) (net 9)))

